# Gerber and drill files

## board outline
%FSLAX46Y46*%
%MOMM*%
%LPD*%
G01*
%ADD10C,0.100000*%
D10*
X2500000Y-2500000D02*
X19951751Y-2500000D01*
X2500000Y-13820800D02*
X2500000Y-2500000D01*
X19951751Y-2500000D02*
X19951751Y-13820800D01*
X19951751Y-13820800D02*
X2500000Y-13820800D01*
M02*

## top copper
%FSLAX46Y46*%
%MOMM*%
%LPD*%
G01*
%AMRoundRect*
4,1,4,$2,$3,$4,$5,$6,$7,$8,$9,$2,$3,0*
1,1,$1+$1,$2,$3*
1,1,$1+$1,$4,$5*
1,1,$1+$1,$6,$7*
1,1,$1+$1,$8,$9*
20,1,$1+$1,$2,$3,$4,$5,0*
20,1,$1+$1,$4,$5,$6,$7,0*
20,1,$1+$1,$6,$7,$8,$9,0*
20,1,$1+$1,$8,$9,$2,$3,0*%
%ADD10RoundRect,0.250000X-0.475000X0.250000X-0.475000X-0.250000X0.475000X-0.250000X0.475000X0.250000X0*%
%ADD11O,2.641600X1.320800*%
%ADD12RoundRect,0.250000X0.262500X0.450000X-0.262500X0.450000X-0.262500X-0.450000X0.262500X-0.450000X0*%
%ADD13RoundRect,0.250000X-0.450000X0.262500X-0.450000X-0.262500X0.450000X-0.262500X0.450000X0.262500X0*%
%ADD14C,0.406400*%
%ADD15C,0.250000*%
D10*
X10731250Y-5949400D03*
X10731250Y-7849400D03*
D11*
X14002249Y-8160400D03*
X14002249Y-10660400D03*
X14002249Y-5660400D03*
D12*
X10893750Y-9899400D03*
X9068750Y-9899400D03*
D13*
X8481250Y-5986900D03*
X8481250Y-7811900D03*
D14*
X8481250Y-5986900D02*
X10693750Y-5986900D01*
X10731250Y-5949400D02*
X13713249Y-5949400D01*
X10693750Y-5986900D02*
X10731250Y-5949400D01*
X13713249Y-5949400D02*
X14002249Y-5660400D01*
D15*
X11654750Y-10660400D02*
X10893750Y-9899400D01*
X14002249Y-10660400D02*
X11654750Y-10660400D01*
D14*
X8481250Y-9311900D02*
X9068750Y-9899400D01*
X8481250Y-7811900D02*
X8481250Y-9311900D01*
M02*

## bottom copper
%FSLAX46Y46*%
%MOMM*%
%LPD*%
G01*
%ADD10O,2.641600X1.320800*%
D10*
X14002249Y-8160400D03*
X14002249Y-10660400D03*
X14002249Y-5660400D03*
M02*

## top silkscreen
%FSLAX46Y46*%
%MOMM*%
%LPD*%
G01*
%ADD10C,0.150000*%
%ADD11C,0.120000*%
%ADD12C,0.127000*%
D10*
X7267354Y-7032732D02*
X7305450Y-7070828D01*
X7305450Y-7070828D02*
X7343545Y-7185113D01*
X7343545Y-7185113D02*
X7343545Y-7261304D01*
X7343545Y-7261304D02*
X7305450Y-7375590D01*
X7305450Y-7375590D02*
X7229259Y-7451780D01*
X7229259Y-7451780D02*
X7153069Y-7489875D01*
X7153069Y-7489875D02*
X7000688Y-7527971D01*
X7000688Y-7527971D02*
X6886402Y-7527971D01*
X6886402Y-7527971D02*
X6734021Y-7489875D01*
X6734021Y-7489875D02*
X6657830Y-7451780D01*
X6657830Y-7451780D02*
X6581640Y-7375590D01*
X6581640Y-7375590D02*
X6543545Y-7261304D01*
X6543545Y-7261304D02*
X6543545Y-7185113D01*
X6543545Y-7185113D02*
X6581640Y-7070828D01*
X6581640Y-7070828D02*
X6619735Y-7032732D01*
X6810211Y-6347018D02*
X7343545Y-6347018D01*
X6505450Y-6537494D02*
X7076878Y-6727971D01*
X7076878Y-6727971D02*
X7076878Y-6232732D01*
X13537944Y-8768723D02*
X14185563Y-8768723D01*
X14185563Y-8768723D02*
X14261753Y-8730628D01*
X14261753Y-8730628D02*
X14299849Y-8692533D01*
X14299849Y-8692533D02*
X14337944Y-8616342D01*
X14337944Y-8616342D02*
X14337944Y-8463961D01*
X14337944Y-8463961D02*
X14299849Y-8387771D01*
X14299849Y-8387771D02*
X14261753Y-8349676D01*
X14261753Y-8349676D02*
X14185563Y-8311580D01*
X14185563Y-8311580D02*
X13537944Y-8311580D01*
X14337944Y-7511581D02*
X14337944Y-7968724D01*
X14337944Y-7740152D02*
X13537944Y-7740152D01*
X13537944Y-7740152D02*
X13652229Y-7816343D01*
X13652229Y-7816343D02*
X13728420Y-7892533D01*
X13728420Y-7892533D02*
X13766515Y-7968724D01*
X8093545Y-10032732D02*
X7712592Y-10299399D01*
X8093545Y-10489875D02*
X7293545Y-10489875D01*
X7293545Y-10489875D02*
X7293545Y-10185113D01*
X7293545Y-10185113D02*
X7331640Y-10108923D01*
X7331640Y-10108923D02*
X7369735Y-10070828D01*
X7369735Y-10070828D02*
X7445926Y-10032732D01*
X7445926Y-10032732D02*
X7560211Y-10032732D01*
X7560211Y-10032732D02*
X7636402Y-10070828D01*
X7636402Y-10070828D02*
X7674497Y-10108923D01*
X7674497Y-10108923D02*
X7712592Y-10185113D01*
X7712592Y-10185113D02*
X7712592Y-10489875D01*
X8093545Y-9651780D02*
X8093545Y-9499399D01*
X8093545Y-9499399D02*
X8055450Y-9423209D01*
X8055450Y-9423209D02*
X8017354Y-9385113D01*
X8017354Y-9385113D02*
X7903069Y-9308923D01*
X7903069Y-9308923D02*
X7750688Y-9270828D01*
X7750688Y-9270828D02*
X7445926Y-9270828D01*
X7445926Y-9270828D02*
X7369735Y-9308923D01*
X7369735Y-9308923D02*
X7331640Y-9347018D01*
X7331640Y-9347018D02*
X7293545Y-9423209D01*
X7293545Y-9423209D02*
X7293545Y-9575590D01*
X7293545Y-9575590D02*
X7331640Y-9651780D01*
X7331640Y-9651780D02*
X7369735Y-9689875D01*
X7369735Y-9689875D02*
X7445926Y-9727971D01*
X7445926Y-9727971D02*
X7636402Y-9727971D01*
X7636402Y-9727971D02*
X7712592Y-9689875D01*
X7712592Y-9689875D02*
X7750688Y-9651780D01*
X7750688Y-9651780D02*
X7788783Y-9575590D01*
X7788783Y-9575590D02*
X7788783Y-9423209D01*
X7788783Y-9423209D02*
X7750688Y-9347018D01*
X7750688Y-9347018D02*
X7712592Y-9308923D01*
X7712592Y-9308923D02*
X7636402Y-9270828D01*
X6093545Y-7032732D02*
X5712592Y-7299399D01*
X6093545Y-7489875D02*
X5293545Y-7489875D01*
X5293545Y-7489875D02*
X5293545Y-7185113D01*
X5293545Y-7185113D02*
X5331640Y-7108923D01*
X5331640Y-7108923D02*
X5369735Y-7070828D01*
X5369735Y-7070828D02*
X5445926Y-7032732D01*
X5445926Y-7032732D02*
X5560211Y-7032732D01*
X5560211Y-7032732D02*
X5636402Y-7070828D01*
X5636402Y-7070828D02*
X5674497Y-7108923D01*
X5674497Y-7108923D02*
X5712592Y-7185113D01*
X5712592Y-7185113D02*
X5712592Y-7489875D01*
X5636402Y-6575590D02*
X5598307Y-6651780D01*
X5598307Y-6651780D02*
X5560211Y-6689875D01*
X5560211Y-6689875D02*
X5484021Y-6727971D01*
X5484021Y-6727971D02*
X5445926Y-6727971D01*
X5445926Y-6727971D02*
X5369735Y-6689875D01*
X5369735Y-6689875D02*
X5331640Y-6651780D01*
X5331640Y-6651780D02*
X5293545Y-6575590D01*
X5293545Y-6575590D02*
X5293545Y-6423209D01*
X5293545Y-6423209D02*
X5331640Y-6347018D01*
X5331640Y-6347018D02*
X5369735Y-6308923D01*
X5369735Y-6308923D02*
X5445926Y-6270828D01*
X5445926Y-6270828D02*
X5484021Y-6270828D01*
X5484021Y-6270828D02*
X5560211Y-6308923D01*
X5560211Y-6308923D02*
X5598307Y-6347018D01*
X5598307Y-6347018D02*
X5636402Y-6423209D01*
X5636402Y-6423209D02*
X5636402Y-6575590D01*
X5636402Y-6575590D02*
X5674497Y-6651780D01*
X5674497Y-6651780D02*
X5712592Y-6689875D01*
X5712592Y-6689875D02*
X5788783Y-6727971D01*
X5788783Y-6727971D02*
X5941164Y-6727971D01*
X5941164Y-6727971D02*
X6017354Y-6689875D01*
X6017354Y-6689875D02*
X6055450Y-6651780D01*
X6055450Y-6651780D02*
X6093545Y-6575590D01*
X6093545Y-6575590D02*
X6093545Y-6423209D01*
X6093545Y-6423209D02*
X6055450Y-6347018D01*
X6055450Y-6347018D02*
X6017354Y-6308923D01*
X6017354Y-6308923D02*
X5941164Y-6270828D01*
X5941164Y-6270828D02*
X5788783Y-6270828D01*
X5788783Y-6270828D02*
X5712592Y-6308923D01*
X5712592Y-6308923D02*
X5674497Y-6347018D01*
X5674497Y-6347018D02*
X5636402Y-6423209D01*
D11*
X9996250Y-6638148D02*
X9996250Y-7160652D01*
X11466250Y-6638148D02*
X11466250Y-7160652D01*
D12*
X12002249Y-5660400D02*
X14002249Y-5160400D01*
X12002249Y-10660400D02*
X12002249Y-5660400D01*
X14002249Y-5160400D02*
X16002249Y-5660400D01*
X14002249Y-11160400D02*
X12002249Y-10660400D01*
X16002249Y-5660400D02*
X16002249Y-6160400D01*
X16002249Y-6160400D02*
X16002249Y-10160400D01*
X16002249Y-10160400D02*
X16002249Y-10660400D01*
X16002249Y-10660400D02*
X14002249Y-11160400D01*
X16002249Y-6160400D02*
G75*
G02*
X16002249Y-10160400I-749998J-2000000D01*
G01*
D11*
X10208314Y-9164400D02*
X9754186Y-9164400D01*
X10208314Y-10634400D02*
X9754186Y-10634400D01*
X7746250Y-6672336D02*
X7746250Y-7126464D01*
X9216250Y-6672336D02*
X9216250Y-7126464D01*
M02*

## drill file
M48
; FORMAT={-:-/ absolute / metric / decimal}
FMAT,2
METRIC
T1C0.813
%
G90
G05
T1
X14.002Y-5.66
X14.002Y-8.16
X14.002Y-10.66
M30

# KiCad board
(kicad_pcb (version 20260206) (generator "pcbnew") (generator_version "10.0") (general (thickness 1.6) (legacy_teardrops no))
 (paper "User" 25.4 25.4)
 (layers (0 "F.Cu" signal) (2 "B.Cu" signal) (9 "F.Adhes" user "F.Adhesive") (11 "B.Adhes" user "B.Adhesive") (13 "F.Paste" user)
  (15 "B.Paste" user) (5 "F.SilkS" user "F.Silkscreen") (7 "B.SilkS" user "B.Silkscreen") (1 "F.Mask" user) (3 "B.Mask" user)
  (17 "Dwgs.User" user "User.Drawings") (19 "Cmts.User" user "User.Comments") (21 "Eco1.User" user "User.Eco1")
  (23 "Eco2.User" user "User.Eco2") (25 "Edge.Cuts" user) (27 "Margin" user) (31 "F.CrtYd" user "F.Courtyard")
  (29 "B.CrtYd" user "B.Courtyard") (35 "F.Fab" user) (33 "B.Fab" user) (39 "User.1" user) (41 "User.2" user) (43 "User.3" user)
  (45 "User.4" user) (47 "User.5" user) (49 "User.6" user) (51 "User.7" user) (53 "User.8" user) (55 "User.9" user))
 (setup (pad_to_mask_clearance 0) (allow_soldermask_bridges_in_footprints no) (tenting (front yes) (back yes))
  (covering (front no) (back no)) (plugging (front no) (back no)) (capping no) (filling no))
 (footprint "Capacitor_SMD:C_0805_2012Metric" (layer "F.Cu") (at 10.73125 6.8994 -90)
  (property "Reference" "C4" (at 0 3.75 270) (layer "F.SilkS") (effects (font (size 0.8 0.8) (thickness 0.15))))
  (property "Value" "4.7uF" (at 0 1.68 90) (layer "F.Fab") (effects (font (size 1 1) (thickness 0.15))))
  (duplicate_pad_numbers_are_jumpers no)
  (fp_line (start -0.261252 0.735) (end 0.261252 0.735) (stroke (width 0.12) (type solid)) (layer "F.SilkS"))
  (fp_line (start -0.261252 -0.735) (end 0.261252 -0.735) (stroke (width 0.12) (type solid)) (layer "F.SilkS"))
  (pad "1" smd roundrect (at -0.95 0 270) (size 1 1.45) (layers "F.Cu" "F.Mask" "F.Paste") (roundrect_rratio 0.25) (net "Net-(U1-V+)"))
  (pad "2" smd roundrect (at 0.95 0 270) (size 1 1.45) (layers "F.Cu" "F.Mask" "F.Paste") (roundrect_rratio 0.25) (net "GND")))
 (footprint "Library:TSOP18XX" (layer "F.Cu") (at 13.975649 8.1592 90)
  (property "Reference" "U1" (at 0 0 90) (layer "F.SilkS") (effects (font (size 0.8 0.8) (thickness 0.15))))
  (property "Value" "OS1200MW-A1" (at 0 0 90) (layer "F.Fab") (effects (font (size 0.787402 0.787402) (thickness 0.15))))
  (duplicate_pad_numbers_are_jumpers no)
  (fp_line (start 2.4988 -1.9734) (end 2.9988 0.0266) (stroke (width 0.127) (type solid)) (layer "F.SilkS"))
  (fp_line (start -2.5012 -1.9734) (end 2.4988 -1.9734) (stroke (width 0.127) (type solid)) (layer "F.SilkS"))
  (fp_line (start 2.9988 0.0266) (end 2.4988 2.0266) (stroke (width 0.127) (type solid)) (layer "F.SilkS"))
  (fp_line (start -3.0012 0.0266) (end -2.5012 -1.9734) (stroke (width 0.127) (type solid)) (layer "F.SilkS"))
  (fp_line (start 2.4988 2.0266) (end 1.9988 2.0266) (stroke (width 0.127) (type solid)) (layer "F.SilkS"))
  (fp_line (start 1.9988 2.0266) (end -2.0012 2.0266) (stroke (width 0.127) (type solid)) (layer "F.SilkS"))
  (fp_line (start -2.0012 2.0266) (end -2.5012 2.0266) (stroke (width 0.127) (type solid)) (layer "F.SilkS"))
  (fp_line (start -2.5012 2.0266) (end -3.0012 0.0266) (stroke (width 0.127) (type solid)) (layer "F.SilkS"))
  (fp_arc (start 1.9988 2.0266) (mid -0.0012 3.412602) (end -2.0012 2.0266) (stroke (width 0.127) (type solid)) (layer "F.SilkS"))
  (pad "GND" thru_hole oval (at -0.0012 0.0266 90) (size 1.3208 2.6416) (drill 0.8128) (layers "*.Cu" "*.Mask") (remove_unused_layers no)
   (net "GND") (solder_mask_margin 0.102))
  (pad "OUT" thru_hole oval (at -2.5012 0.0266 90) (size 1.3208 2.6416) (drill 0.8128) (layers "*.Cu" "*.Mask") (remove_unused_layers no)
   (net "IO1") (solder_mask_margin 0.102))
  (pad "VCC" thru_hole oval (at 2.4988 0.0266 90) (size 1.3208 2.6416) (drill 0.8128) (layers "*.Cu" "*.Mask") (remove_unused_layers no)
   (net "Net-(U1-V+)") (solder_mask_margin 0.102)))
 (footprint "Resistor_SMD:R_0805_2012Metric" (layer "F.Cu") (at 9.98125 9.8994 180)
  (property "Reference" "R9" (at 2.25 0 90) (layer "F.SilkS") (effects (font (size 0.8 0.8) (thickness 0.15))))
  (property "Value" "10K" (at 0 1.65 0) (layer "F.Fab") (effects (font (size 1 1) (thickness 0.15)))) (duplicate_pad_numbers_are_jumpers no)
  (fp_line (start -0.227064 0.735) (end 0.227064 0.735) (stroke (width 0.12) (type solid)) (layer "F.SilkS"))
  (fp_line (start -0.227064 -0.735) (end 0.227064 -0.735) (stroke (width 0.12) (type solid)) (layer "F.SilkS"))
  (pad "1" smd roundrect (at -0.9125 0 180) (size 1.025 1.4) (layers "F.Cu" "F.Mask" "F.Paste") (roundrect_rratio 0.243902439) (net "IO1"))
  (pad "2" smd roundrect (at 0.9125 0 180) (size 1.025 1.4) (layers "F.Cu" "F.Mask" "F.Paste") (roundrect_rratio 0.243902439) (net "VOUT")))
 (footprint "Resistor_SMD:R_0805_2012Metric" (layer "F.Cu") (at 8.48125 6.8994 -90)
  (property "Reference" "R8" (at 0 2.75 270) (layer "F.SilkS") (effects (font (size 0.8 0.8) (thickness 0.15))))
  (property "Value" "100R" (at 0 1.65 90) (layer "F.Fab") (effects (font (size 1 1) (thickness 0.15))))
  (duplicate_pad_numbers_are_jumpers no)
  (fp_line (start -0.227064 0.735) (end 0.227064 0.735) (stroke (width 0.12) (type solid)) (layer "F.SilkS"))
  (fp_line (start -0.227064 -0.735) (end 0.227064 -0.735) (stroke (width 0.12) (type solid)) (layer "F.SilkS"))
  (pad "1" smd roundrect (at -0.9125 0 270) (size 1.025 1.4) (layers "F.Cu" "F.Mask" "F.Paste") (roundrect_rratio 0.243902439)
   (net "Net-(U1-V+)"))
  (pad "2" smd roundrect (at 0.9125 0 270) (size 1.025 1.4) (layers "F.Cu" "F.Mask" "F.Paste") (roundrect_rratio 0.243902439) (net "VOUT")))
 (gr_line (start 2.5 2.5) (end 19.951751 2.5) (stroke (width 0.1) (type default)) (layer "Edge.Cuts"))
 (gr_line (start 2.5 13.8208) (end 2.5 2.5) (stroke (width 0.1) (type default)) (layer "Edge.Cuts"))
 (gr_line (start 19.951751 2.5) (end 19.951751 13.8208) (stroke (width 0.1) (type default)) (layer "Edge.Cuts"))
 (gr_line (start 19.951751 13.8208) (end 2.5 13.8208) (stroke (width 0.1) (type default)) (layer "Edge.Cuts"))
 (segment (start 8.48125 5.9869) (end 10.69375 5.9869) (width 0.4064) (layer "F.Cu") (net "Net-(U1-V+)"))
 (segment (start 10.73125 5.9494) (end 13.713249 5.9494) (width 0.4064) (layer "F.Cu") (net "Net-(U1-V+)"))
 (segment (start 10.69375 5.9869) (end 10.73125 5.9494) (width 0.4064) (layer "F.Cu") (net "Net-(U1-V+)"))
 (segment (start 13.713249 5.9494) (end 14.002249 5.6604) (width 0.4064) (layer "F.Cu") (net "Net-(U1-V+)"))
 (segment (start 11.65475 10.6604) (end 10.89375 9.8994) (width 0.25) (layer "F.Cu") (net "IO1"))
 (segment (start 14.002249 10.6604) (end 11.65475 10.6604) (width 0.25) (layer "F.Cu") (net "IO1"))
 (segment (start 8.48125 9.3119) (end 9.06875 9.8994) (width 0.4064) (layer "F.Cu") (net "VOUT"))
 (segment (start 8.48125 7.8119) (end 8.48125 9.3119) (width 0.4064) (layer "F.Cu") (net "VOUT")))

